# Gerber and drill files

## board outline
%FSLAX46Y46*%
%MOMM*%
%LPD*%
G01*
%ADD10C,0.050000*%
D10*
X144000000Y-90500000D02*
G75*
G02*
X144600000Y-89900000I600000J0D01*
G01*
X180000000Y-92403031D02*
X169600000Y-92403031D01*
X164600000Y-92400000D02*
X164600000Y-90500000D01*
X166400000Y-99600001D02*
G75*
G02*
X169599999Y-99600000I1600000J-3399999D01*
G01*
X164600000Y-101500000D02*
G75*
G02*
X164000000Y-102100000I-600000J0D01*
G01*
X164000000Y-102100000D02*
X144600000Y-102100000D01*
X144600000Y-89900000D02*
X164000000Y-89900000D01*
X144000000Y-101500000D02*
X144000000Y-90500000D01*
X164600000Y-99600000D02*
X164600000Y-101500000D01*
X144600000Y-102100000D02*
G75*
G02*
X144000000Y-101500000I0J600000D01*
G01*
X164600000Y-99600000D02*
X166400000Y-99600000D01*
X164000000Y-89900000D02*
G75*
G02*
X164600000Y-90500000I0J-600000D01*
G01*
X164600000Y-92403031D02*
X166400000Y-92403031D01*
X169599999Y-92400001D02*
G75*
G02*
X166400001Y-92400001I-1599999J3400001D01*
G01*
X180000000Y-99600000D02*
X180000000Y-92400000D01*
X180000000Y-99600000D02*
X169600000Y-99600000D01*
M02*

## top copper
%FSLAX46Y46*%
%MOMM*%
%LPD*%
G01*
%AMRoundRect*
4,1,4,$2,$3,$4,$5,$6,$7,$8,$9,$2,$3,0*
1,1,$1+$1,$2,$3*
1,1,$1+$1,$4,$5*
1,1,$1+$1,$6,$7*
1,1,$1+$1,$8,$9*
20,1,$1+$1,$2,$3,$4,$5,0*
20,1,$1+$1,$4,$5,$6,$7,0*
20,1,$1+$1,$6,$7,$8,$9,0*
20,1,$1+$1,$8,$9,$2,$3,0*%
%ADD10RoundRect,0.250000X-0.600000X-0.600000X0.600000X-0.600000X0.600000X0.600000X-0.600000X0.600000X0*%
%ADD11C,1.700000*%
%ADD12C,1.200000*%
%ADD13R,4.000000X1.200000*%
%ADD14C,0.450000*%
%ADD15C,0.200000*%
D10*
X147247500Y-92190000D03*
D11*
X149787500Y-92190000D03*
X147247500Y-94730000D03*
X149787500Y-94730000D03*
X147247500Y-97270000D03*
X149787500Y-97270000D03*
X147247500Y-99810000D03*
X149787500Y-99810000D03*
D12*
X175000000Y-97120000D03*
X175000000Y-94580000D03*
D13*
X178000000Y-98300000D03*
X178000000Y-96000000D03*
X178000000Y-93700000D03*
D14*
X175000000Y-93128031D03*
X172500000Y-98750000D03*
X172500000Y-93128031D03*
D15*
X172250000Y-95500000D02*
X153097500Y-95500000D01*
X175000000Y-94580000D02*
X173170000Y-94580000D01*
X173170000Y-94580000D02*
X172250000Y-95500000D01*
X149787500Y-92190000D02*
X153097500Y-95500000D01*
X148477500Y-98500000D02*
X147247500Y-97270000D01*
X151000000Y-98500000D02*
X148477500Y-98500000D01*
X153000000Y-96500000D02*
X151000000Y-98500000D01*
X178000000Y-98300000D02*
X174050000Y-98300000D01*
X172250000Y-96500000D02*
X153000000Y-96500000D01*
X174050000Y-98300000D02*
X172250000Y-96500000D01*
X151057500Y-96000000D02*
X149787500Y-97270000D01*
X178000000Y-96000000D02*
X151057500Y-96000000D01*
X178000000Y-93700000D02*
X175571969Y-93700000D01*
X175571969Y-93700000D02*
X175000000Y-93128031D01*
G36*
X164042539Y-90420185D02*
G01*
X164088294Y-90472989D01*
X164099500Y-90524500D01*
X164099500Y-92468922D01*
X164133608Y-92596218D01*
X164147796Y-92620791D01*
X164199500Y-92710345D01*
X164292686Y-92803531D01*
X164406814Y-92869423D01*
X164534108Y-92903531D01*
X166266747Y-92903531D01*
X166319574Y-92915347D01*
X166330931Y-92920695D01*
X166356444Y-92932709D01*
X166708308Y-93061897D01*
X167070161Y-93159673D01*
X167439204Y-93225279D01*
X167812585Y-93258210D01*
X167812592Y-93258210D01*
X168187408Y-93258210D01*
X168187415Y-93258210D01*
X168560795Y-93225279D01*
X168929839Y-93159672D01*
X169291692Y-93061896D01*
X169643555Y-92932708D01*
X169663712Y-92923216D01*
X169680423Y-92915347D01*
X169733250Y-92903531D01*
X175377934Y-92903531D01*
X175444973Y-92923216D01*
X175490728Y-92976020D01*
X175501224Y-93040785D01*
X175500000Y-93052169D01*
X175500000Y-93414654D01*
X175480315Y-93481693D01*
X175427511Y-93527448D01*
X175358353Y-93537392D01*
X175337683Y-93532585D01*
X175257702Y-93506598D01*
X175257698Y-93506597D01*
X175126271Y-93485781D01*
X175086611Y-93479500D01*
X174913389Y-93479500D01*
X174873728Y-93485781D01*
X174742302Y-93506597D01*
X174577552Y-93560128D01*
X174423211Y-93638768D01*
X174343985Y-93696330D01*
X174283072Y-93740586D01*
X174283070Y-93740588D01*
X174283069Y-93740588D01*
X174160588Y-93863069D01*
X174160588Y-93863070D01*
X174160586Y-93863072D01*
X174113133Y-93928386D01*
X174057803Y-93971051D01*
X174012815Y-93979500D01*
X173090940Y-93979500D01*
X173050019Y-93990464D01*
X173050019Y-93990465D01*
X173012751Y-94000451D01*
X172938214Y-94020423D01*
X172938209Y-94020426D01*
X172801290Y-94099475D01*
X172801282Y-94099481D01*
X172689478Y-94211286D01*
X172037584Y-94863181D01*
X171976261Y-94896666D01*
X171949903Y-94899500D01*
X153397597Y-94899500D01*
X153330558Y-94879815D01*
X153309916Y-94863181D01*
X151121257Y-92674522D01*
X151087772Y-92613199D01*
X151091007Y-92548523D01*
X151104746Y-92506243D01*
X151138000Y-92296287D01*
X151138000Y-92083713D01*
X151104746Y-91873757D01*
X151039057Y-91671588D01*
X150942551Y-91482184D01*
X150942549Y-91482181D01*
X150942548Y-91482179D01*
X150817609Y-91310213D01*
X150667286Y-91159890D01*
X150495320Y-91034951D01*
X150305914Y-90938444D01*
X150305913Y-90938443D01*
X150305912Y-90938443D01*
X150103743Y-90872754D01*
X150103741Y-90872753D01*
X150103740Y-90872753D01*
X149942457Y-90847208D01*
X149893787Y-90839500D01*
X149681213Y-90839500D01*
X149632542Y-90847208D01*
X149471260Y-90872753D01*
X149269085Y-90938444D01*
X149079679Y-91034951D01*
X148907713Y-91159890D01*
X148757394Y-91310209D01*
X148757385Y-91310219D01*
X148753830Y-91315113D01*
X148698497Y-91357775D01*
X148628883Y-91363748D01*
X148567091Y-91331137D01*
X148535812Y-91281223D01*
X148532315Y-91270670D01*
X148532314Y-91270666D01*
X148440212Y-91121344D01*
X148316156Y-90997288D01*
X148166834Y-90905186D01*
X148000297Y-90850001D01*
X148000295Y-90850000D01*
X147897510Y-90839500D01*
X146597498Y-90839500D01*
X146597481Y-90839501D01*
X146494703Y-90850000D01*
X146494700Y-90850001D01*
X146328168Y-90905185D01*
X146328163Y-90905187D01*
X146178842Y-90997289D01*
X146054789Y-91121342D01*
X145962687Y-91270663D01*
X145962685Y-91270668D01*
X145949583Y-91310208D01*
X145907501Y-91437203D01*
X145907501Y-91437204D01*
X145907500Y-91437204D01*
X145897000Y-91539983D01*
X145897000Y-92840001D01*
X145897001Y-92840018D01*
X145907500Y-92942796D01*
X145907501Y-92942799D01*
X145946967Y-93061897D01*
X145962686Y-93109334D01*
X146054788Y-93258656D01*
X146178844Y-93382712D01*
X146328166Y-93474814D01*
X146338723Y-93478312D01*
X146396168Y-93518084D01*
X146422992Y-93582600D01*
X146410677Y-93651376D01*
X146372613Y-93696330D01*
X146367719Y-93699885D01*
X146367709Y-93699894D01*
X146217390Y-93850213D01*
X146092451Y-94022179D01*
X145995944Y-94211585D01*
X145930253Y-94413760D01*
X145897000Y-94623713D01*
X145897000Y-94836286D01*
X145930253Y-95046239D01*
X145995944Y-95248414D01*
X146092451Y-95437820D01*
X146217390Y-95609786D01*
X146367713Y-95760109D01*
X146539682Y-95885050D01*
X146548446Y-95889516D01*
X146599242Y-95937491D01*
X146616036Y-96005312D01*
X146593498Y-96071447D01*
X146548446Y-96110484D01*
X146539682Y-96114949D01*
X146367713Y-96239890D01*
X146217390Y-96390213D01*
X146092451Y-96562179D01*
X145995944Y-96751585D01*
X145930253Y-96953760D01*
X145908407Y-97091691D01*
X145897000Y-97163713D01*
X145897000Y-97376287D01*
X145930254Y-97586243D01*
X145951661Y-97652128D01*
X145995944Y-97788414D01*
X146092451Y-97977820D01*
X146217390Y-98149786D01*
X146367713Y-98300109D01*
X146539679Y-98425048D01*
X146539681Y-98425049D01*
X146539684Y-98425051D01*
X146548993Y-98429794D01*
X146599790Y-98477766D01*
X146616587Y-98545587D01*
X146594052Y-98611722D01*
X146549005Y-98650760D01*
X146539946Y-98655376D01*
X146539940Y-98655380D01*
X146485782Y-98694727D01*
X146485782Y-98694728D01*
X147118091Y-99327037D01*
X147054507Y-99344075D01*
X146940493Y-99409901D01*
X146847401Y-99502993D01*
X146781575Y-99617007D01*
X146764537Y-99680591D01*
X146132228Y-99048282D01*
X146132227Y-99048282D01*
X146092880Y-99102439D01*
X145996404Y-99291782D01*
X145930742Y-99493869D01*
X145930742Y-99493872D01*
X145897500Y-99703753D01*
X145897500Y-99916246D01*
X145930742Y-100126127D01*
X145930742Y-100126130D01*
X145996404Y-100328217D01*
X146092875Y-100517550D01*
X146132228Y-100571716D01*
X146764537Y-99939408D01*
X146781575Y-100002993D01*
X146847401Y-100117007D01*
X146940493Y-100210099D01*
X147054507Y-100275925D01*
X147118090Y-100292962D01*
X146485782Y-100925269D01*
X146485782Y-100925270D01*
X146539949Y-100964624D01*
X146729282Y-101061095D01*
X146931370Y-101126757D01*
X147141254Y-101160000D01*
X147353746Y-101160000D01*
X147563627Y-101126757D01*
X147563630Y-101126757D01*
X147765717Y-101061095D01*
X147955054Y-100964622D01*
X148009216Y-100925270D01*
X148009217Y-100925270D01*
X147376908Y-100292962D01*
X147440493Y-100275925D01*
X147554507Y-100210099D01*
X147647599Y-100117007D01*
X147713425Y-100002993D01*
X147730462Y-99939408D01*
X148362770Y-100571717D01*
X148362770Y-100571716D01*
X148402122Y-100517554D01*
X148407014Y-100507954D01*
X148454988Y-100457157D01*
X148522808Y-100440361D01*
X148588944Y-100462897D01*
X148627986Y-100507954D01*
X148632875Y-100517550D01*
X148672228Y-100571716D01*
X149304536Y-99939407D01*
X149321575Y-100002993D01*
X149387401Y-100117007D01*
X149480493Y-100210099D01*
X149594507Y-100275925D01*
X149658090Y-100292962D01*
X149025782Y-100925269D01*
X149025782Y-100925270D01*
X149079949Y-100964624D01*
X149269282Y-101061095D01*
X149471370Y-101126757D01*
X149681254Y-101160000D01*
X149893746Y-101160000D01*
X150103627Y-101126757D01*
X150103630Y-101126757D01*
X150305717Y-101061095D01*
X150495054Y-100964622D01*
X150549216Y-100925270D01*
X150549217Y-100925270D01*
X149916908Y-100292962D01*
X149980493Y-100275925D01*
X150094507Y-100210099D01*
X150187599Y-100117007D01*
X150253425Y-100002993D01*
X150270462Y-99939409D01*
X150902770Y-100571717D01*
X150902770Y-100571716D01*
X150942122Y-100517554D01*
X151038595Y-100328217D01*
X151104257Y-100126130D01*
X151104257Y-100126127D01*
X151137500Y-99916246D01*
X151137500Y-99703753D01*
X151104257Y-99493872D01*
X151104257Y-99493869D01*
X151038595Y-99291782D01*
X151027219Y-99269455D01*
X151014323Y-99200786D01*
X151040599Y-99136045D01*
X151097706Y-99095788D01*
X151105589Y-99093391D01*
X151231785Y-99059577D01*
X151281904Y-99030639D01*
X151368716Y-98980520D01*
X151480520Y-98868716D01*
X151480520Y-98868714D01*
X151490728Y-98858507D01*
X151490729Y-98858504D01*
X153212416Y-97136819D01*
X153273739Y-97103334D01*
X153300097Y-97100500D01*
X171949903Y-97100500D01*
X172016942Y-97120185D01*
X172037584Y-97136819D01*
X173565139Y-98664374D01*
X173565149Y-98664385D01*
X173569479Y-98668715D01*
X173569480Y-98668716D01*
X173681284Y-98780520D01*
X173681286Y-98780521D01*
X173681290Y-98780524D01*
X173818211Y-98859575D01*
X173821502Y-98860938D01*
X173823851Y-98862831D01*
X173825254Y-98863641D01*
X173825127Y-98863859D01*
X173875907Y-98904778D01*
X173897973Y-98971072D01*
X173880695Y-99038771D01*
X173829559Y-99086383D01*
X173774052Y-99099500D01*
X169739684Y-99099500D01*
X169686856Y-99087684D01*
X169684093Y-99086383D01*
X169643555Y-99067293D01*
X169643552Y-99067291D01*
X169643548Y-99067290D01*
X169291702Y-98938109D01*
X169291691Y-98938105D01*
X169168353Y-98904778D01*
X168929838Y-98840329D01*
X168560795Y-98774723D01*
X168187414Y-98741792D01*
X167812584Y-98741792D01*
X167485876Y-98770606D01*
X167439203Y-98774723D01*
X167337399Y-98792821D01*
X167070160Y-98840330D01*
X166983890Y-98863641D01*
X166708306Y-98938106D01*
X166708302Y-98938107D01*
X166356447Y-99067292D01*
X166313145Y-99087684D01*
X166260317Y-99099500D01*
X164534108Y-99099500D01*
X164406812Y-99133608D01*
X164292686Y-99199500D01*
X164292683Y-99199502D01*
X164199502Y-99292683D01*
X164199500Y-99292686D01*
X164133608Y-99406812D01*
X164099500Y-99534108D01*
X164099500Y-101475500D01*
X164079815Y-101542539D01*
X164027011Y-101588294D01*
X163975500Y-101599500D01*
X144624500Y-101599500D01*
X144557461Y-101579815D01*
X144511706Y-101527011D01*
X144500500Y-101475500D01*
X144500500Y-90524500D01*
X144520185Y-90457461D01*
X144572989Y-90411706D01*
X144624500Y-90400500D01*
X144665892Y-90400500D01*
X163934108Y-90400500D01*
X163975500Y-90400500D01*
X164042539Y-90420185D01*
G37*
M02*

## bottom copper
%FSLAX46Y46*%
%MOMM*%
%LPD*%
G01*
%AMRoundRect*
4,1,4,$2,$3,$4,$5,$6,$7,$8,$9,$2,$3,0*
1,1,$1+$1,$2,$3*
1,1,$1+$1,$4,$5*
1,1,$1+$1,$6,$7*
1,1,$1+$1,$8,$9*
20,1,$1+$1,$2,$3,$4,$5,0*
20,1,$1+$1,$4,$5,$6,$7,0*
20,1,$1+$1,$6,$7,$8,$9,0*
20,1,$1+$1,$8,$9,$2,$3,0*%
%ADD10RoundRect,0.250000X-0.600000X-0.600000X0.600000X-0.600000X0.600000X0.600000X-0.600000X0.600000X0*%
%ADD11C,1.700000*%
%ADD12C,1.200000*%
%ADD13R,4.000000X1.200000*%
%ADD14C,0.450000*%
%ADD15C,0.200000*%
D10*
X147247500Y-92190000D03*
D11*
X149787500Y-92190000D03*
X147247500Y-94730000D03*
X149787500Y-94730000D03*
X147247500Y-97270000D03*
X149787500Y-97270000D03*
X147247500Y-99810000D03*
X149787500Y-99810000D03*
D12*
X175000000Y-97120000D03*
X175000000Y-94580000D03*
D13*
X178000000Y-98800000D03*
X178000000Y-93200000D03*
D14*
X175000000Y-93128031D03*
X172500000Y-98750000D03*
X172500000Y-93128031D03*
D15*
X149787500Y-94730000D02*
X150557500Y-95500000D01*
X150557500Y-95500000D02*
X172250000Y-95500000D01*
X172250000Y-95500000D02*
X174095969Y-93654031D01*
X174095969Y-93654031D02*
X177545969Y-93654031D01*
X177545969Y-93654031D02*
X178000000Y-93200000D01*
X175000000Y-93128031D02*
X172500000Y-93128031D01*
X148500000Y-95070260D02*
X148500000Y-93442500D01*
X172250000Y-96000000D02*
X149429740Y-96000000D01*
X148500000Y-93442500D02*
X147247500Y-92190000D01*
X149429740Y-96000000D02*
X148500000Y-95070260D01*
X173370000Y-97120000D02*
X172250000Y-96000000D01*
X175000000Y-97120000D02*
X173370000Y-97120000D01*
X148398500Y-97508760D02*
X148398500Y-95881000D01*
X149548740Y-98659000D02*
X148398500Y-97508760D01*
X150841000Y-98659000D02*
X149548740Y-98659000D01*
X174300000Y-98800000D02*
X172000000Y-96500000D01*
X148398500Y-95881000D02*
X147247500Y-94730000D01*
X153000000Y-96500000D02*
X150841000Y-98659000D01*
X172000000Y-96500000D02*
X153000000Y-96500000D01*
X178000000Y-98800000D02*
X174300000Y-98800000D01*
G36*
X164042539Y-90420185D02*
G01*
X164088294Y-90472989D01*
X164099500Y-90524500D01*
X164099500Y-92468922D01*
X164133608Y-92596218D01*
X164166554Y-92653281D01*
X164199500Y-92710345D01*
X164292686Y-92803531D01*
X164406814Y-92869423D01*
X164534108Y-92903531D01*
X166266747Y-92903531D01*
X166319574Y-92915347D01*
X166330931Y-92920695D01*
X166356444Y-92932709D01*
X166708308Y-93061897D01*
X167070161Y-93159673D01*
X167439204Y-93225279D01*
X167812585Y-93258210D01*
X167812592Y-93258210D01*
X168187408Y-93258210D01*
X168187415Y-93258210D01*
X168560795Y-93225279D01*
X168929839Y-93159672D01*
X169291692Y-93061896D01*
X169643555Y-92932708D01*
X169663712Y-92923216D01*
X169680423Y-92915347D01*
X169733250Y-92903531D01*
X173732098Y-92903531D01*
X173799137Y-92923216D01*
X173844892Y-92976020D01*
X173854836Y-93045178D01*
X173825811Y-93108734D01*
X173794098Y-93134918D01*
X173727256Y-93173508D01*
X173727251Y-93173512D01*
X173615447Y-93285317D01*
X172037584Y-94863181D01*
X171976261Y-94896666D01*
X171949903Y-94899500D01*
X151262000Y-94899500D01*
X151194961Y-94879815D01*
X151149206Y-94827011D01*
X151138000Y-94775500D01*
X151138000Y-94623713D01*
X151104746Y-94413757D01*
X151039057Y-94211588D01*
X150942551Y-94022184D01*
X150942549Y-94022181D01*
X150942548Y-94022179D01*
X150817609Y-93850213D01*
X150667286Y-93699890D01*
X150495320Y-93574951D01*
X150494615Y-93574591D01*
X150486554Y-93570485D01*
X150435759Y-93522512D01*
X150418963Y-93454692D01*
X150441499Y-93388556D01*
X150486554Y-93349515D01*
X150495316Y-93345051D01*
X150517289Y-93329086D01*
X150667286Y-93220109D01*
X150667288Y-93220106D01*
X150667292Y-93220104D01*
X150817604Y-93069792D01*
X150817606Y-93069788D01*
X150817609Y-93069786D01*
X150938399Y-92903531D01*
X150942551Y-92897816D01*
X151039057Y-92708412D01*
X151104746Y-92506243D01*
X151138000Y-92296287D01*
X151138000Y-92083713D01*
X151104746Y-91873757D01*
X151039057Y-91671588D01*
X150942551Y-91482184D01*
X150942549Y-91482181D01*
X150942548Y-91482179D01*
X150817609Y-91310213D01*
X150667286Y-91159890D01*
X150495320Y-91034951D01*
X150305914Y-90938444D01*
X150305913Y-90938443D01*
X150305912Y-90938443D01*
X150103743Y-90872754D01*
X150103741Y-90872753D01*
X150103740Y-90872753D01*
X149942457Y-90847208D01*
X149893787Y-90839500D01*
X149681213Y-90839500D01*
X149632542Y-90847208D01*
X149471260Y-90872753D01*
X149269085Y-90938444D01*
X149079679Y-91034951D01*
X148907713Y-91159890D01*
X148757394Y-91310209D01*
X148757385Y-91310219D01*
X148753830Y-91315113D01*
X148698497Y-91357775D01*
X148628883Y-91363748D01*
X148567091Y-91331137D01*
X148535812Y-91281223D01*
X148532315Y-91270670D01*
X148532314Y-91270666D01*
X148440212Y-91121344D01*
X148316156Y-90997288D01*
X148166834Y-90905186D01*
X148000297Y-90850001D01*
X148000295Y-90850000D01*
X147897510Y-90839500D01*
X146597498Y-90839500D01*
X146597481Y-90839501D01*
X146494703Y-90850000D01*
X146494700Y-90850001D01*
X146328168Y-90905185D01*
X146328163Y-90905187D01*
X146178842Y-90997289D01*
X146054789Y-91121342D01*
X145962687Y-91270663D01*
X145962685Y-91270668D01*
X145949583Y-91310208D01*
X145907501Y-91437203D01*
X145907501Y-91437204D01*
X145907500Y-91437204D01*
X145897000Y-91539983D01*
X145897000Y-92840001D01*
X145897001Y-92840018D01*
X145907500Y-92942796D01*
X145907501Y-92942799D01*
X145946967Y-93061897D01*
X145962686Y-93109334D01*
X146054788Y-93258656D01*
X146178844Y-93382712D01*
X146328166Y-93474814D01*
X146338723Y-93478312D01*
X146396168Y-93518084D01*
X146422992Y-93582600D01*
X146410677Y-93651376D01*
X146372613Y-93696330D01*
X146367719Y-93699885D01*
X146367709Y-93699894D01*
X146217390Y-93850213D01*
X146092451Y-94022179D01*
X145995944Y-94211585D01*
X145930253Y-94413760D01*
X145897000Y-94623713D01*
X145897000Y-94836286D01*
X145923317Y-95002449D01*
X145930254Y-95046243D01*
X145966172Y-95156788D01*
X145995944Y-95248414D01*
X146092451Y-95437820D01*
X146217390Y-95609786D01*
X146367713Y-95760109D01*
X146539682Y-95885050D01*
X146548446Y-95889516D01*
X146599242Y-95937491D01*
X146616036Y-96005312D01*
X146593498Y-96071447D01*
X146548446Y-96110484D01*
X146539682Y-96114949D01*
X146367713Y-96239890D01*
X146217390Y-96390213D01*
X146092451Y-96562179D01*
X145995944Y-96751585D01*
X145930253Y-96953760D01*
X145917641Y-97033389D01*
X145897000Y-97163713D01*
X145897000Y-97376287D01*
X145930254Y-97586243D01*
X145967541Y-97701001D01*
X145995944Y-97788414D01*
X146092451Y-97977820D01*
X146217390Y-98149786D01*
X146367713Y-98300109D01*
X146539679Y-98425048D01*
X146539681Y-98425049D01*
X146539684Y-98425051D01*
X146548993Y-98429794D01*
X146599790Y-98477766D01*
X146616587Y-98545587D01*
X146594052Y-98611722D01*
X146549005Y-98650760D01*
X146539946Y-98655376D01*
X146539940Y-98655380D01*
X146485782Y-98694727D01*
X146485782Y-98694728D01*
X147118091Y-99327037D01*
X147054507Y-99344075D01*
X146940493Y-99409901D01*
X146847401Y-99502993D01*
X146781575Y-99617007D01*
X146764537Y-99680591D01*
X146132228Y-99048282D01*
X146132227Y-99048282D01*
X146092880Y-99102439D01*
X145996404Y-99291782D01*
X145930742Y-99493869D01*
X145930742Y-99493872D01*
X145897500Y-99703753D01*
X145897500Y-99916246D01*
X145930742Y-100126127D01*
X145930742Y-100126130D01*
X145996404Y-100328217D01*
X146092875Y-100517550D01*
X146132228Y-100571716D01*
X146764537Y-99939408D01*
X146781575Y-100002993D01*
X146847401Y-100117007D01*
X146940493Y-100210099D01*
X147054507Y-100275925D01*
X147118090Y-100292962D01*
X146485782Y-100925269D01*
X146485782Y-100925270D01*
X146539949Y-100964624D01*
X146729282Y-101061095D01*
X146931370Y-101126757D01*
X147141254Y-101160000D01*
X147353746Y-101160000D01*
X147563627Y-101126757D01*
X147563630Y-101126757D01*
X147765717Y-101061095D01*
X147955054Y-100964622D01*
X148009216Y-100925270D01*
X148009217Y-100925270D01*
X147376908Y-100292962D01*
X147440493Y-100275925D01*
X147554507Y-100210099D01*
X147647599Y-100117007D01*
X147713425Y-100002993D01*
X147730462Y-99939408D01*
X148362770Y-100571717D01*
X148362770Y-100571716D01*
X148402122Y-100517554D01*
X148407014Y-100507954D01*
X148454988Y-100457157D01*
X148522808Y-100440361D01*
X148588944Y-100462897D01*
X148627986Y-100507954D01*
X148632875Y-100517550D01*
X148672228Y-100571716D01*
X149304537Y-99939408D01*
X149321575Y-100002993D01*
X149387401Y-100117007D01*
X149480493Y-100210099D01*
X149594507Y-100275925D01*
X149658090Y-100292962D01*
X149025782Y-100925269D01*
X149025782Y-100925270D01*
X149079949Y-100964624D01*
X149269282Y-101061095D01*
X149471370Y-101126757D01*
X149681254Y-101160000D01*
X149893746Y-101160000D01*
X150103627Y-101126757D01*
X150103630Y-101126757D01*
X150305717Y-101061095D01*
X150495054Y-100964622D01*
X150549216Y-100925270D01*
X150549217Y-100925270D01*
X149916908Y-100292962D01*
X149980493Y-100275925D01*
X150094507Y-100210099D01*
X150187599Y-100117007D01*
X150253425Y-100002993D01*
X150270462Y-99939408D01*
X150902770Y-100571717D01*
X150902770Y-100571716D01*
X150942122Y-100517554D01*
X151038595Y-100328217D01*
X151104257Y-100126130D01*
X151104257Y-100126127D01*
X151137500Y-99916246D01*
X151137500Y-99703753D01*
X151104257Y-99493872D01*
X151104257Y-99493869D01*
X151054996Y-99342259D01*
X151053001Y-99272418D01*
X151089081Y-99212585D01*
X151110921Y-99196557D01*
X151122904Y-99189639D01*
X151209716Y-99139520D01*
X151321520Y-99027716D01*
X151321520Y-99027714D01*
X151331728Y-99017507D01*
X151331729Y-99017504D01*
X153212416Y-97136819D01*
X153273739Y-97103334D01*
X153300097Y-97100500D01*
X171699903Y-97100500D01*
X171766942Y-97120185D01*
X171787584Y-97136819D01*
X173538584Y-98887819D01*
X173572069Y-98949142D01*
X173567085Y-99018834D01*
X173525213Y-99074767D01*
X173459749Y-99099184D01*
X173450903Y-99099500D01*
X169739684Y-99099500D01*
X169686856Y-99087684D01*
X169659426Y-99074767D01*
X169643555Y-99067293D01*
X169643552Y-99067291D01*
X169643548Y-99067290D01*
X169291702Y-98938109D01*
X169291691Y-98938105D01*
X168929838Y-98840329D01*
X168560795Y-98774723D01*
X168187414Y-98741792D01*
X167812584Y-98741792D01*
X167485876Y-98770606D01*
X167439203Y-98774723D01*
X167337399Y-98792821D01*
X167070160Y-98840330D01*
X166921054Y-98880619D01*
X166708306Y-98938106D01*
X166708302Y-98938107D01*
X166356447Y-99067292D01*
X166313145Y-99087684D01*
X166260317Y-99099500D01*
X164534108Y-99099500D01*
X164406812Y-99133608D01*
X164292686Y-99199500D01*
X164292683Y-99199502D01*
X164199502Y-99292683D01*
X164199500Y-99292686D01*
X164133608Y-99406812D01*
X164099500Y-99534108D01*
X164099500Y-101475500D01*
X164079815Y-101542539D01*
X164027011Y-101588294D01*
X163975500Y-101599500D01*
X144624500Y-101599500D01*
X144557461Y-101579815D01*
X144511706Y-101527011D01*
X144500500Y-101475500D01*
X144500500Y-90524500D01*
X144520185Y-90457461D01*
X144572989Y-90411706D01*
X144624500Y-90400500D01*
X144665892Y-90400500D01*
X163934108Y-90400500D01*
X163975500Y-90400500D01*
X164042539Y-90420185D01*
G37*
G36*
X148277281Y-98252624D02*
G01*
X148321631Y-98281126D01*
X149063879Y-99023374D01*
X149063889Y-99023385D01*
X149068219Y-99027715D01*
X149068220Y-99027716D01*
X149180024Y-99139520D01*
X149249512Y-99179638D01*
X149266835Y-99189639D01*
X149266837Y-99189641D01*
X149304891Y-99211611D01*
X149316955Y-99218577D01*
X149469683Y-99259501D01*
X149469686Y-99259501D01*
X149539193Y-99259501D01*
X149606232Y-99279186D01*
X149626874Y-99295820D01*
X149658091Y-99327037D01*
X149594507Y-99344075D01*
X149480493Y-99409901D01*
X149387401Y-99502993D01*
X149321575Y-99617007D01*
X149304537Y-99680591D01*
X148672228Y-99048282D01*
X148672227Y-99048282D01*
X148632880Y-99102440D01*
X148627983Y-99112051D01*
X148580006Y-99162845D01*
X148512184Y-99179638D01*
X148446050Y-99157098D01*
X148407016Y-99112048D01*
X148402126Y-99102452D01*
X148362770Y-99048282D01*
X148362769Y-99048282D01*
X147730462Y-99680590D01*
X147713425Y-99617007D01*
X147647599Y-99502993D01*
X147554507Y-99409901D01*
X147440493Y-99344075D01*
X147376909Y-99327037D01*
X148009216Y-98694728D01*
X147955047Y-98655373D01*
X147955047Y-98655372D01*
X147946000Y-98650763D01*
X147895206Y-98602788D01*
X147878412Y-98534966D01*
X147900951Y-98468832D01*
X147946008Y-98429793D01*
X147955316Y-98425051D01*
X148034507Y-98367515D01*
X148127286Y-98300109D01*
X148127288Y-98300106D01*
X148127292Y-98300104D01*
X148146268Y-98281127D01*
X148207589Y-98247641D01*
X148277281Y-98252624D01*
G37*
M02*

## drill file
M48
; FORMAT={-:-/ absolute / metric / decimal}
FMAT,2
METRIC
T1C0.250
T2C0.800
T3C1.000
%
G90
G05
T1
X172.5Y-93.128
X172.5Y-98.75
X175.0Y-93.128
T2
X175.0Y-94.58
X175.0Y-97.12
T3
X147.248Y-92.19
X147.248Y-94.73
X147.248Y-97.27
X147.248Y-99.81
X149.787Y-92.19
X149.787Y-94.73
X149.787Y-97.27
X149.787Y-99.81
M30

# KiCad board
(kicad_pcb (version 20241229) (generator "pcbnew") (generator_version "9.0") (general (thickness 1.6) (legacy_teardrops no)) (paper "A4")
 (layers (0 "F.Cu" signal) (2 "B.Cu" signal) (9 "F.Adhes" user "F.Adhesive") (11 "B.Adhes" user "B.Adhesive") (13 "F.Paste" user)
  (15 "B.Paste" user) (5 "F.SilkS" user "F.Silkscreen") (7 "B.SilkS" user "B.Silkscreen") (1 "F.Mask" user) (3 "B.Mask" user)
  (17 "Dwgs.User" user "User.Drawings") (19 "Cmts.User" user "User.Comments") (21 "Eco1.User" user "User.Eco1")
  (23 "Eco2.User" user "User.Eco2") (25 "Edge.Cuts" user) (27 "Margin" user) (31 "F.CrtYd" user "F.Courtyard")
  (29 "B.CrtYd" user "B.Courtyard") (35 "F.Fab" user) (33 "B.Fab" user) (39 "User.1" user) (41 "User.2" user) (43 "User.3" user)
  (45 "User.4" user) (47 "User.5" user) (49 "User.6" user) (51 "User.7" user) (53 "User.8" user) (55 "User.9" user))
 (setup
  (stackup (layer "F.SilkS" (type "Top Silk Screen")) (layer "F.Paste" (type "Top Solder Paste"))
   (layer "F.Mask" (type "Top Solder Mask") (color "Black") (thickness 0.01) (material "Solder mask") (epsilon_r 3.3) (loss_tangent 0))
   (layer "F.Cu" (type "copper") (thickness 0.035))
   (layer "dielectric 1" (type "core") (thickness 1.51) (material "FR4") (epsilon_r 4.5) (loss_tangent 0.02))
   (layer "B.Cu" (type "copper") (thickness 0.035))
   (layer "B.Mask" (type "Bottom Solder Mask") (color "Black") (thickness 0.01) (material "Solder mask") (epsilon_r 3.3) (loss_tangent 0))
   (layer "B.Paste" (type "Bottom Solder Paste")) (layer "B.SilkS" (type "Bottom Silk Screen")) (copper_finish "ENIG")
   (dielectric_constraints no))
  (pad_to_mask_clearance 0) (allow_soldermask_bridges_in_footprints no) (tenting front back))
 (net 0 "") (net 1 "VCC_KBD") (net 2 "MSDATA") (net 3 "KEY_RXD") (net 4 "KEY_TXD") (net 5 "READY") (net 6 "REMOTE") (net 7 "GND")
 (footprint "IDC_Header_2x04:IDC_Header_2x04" (layer "F.Cu") (at 147.2475 92.19)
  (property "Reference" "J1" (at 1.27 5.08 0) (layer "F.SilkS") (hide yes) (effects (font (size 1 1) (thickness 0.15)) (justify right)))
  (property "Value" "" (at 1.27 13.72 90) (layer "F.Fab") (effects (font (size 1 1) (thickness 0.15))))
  (pad "1" thru_hole roundrect (at 0 0) (size 1.7 1.7) (drill 1) (layers "*.Cu" "*.Mask") (remove_unused_layers no)
   (roundrect_rratio 0.147059) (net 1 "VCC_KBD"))
  (pad "2" thru_hole circle (at 2.54 0) (size 1.7 1.7) (drill 1) (layers "*.Cu" "*.Mask") (remove_unused_layers no) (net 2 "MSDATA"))
  (pad "3" thru_hole circle (at 0 2.54) (size 1.7 1.7) (drill 1) (layers "*.Cu" "*.Mask") (remove_unused_layers no) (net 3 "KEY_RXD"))
  (pad "4" thru_hole circle (at 2.54 2.54) (size 1.7 1.7) (drill 1) (layers "*.Cu" "*.Mask") (remove_unused_layers no) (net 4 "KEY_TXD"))
  (pad "5" thru_hole circle (at 0 5.08) (size 1.7 1.7) (drill 1) (layers "*.Cu" "*.Mask") (remove_unused_layers no) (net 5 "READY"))
  (pad "6" thru_hole circle (at 2.54 5.08) (size 1.7 1.7) (drill 1) (layers "*.Cu" "*.Mask") (remove_unused_layers no) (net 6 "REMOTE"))
  (pad "7" thru_hole circle (at 0 7.62) (size 1.7 1.7) (drill 1) (layers "*.Cu" "*.Mask") (remove_unused_layers no) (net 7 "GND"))
  (pad "8" thru_hole circle (at 2.54 7.62) (size 1.7 1.7) (drill 1) (layers "*.Cu" "*.Mask") (remove_unused_layers no) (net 7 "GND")))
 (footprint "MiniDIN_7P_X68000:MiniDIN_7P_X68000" (layer "F.Cu") (at 180 96)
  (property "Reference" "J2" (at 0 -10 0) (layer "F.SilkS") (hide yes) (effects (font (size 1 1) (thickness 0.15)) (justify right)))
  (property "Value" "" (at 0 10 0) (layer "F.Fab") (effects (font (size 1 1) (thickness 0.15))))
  (pad "1" thru_hole circle (at -5 1.12) (size 1.2 1.2) (drill 0.8) (layers "*.Cu" "*.Mask") (remove_unused_layers no) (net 1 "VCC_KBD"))
  (pad "2" thru_hole circle (at -5 -1.42) (size 1.2 1.2) (drill 0.8) (layers "*.Cu" "*.Mask") (remove_unused_layers no) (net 2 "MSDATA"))
  (pad "3" connect rect (at -2 2.8) (size 4 1.2) (layers "B.Cu" "B.Mask") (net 3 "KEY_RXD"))
  (pad "4" connect rect (at -2 -2.8) (size 4 1.2) (layers "B.Cu" "B.Mask") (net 4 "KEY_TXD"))
  (pad "5" connect rect (at -2 2.3) (size 4 1.2) (layers "F.Cu" "F.Mask") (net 5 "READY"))
  (pad "6" connect rect (at -2 0) (size 4 1.2) (layers "F.Cu" "F.Mask") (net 6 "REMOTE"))
  (pad "7" connect rect (at -2 -2.3) (size 4 1.2) (layers "F.Cu" "F.Mask") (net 7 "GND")))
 (gr_arc (start 144 90.5) (mid 144.175736 90.075736) (end 144.6 89.9) (stroke (width 0.05) (type default)) (layer "Edge.Cuts"))
 (gr_line (start 180 92.403031) (end 169.6 92.403031) (stroke (width 0.05) (type default)) (layer "Edge.Cuts"))
 (gr_line (start 164.6 92.4) (end 164.6 90.5) (stroke (width 0.05) (type default)) (layer "Edge.Cuts"))
 (gr_arc (start 166.4 99.600001) (mid 167.999999 99.242342) (end 169.599999 99.6) (stroke (width 0.05) (type default)) (layer "Edge.Cuts"))
 (gr_arc (start 164.6 101.5) (mid 164.424264 101.924264) (end 164 102.1) (stroke (width 0.05) (type default)) (layer "Edge.Cuts"))
 (gr_line (start 164 102.1) (end 144.6 102.1) (stroke (width 0.05) (type default)) (layer "Edge.Cuts"))
 (gr_line (start 144.6 89.9) (end 164 89.9) (stroke (width 0.05) (type default)) (layer "Edge.Cuts"))
 (gr_line (start 144 101.5) (end 144 90.5) (stroke (width 0.05) (type default)) (layer "Edge.Cuts"))
 (gr_line (start 164.6 99.6) (end 164.6 101.5) (stroke (width 0.05) (type default)) (layer "Edge.Cuts"))
 (gr_arc (start 144.6 102.1) (mid 144.175736 101.924264) (end 144 101.5) (stroke (width 0.05) (type default)) (layer "Edge.Cuts"))
 (gr_line (start 164.6 99.6) (end 166.4 99.6) (stroke (width 0.05) (type default)) (layer "Edge.Cuts"))
 (gr_arc (start 164 89.9) (mid 164.424264 90.075736) (end 164.6 90.5) (stroke (width 0.05) (type default)) (layer "Edge.Cuts"))
 (gr_line (start 164.6 92.403031) (end 166.4 92.403031) (stroke (width 0.05) (type default)) (layer "Edge.Cuts"))
 (gr_arc (start 169.599999 92.400001) (mid 168 92.75766) (end 166.4 92.400002) (stroke (width 0.05) (type default)) (layer "Edge.Cuts"))
 (gr_line (start 180 99.6) (end 180 92.4) (stroke (width 0.05) (type default)) (layer "Edge.Cuts"))
 (gr_line (start 180 99.6) (end 169.6 99.6) (stroke (width 0.05) (type default)) (layer "Edge.Cuts"))
 (segment (start 172.25 95.5) (end 153.0975 95.5) (width 0.2) (layer "F.Cu") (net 2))
 (segment (start 175 94.58) (end 173.17 94.58) (width 0.2) (layer "F.Cu") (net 2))
 (segment (start 173.17 94.58) (end 172.25 95.5) (width 0.2) (layer "F.Cu") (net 2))
 (segment (start 149.7875 92.19) (end 153.0975 95.5) (width 0.2) (layer "F.Cu") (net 2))
 (segment (start 149.7875 94.73) (end 150.5575 95.5) (width 0.2) (layer "B.Cu") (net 4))
 (segment (start 150.5575 95.5) (end 172.25 95.5) (width 0.2) (layer "B.Cu") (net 4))
 (segment (start 172.25 95.5) (end 174.095969 93.654031) (width 0.2) (layer "B.Cu") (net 4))
 (segment (start 174.095969 93.654031) (end 177.545969 93.654031) (width 0.2) (layer "B.Cu") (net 4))
 (segment (start 177.545969 93.654031) (end 178 93.2) (width 0.2) (layer "B.Cu") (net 4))
 (segment (start 148.4775 98.5) (end 147.2475 97.27) (width 0.2) (layer "F.Cu") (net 5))
 (segment (start 151 98.5) (end 148.4775 98.5) (width 0.2) (layer "F.Cu") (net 5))
 (segment (start 153 96.5) (end 151 98.5) (width 0.2) (layer "F.Cu") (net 5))
 (segment (start 178 98.3) (end 174.05 98.3) (width 0.2) (layer "F.Cu") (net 5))
 (segment (start 172.25 96.5) (end 153 96.5) (width 0.2) (layer "F.Cu") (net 5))
 (segment (start 174.05 98.3) (end 172.25 96.5) (width 0.2) (layer "F.Cu") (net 5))
 (segment (start 151.0575 96) (end 149.7875 97.27) (width 0.2) (layer "F.Cu") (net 6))
 (segment (start 178 96) (end 151.0575 96) (width 0.2) (layer "F.Cu") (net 6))
 (segment (start 178 93.7) (end 175.571969 93.7) (width 0.2) (layer "F.Cu") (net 7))
 (segment (start 175.571969 93.7) (end 175 93.128031) (width 0.2) (layer "F.Cu") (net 7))
 (via (at 175 93.128031) (size 0.45) (drill 0.25) (layers "F.Cu" "B.Cu") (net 7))
 (via (at 172.5 98.75) (size 0.45) (drill 0.25) (layers "F.Cu" "B.Cu") (free yes) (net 7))
 (via (at 172.5 93.128031) (size 0.45) (drill 0.25) (layers "F.Cu" "B.Cu") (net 7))
 (segment (start 175 93.128031) (end 172.5 93.128031) (width 0.2) (layer "B.Cu") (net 7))
 (segment (start 148.5 95.07026) (end 148.5 93.4425) (width 0.2) (layer "B.Cu") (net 1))
 (segment (start 172.25 96) (end 149.42974 96) (width 0.2) (layer "B.Cu") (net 1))
 (segment (start 148.5 93.4425) (end 147.2475 92.19) (width 0.2) (layer "B.Cu") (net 1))
 (segment (start 149.42974 96) (end 148.5 95.07026) (width 0.2) (layer "B.Cu") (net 1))
 (segment (start 173.37 97.12) (end 172.25 96) (width 0.2) (layer "B.Cu") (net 1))
 (segment (start 175 97.12) (end 173.37 97.12) (width 0.2) (layer "B.Cu") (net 1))
 (segment (start 148.3985 97.50876) (end 148.3985 95.881) (width 0.2) (layer "B.Cu") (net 3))
 (segment (start 149.54874 98.659) (end 148.3985 97.50876) (width 0.2) (layer "B.Cu") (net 3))
 (segment (start 150.841 98.659) (end 149.54874 98.659) (width 0.2) (layer "B.Cu") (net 3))
 (segment (start 174.3 98.8) (end 172 96.5) (width 0.2) (layer "B.Cu") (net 3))
 (segment (start 148.3985 95.881) (end 147.2475 94.73) (width 0.2) (layer "B.Cu") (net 3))
 (segment (start 153 96.5) (end 150.841 98.659) (width 0.2) (layer "B.Cu") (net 3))
 (segment (start 172 96.5) (end 153 96.5) (width 0.2) (layer "B.Cu") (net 3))
 (segment (start 178 98.8) (end 174.3 98.8) (width 0.2) (layer "B.Cu") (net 3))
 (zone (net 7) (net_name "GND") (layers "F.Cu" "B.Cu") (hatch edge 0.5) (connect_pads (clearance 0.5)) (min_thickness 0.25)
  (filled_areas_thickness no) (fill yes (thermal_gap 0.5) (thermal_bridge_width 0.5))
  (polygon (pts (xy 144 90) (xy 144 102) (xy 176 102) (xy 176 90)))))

